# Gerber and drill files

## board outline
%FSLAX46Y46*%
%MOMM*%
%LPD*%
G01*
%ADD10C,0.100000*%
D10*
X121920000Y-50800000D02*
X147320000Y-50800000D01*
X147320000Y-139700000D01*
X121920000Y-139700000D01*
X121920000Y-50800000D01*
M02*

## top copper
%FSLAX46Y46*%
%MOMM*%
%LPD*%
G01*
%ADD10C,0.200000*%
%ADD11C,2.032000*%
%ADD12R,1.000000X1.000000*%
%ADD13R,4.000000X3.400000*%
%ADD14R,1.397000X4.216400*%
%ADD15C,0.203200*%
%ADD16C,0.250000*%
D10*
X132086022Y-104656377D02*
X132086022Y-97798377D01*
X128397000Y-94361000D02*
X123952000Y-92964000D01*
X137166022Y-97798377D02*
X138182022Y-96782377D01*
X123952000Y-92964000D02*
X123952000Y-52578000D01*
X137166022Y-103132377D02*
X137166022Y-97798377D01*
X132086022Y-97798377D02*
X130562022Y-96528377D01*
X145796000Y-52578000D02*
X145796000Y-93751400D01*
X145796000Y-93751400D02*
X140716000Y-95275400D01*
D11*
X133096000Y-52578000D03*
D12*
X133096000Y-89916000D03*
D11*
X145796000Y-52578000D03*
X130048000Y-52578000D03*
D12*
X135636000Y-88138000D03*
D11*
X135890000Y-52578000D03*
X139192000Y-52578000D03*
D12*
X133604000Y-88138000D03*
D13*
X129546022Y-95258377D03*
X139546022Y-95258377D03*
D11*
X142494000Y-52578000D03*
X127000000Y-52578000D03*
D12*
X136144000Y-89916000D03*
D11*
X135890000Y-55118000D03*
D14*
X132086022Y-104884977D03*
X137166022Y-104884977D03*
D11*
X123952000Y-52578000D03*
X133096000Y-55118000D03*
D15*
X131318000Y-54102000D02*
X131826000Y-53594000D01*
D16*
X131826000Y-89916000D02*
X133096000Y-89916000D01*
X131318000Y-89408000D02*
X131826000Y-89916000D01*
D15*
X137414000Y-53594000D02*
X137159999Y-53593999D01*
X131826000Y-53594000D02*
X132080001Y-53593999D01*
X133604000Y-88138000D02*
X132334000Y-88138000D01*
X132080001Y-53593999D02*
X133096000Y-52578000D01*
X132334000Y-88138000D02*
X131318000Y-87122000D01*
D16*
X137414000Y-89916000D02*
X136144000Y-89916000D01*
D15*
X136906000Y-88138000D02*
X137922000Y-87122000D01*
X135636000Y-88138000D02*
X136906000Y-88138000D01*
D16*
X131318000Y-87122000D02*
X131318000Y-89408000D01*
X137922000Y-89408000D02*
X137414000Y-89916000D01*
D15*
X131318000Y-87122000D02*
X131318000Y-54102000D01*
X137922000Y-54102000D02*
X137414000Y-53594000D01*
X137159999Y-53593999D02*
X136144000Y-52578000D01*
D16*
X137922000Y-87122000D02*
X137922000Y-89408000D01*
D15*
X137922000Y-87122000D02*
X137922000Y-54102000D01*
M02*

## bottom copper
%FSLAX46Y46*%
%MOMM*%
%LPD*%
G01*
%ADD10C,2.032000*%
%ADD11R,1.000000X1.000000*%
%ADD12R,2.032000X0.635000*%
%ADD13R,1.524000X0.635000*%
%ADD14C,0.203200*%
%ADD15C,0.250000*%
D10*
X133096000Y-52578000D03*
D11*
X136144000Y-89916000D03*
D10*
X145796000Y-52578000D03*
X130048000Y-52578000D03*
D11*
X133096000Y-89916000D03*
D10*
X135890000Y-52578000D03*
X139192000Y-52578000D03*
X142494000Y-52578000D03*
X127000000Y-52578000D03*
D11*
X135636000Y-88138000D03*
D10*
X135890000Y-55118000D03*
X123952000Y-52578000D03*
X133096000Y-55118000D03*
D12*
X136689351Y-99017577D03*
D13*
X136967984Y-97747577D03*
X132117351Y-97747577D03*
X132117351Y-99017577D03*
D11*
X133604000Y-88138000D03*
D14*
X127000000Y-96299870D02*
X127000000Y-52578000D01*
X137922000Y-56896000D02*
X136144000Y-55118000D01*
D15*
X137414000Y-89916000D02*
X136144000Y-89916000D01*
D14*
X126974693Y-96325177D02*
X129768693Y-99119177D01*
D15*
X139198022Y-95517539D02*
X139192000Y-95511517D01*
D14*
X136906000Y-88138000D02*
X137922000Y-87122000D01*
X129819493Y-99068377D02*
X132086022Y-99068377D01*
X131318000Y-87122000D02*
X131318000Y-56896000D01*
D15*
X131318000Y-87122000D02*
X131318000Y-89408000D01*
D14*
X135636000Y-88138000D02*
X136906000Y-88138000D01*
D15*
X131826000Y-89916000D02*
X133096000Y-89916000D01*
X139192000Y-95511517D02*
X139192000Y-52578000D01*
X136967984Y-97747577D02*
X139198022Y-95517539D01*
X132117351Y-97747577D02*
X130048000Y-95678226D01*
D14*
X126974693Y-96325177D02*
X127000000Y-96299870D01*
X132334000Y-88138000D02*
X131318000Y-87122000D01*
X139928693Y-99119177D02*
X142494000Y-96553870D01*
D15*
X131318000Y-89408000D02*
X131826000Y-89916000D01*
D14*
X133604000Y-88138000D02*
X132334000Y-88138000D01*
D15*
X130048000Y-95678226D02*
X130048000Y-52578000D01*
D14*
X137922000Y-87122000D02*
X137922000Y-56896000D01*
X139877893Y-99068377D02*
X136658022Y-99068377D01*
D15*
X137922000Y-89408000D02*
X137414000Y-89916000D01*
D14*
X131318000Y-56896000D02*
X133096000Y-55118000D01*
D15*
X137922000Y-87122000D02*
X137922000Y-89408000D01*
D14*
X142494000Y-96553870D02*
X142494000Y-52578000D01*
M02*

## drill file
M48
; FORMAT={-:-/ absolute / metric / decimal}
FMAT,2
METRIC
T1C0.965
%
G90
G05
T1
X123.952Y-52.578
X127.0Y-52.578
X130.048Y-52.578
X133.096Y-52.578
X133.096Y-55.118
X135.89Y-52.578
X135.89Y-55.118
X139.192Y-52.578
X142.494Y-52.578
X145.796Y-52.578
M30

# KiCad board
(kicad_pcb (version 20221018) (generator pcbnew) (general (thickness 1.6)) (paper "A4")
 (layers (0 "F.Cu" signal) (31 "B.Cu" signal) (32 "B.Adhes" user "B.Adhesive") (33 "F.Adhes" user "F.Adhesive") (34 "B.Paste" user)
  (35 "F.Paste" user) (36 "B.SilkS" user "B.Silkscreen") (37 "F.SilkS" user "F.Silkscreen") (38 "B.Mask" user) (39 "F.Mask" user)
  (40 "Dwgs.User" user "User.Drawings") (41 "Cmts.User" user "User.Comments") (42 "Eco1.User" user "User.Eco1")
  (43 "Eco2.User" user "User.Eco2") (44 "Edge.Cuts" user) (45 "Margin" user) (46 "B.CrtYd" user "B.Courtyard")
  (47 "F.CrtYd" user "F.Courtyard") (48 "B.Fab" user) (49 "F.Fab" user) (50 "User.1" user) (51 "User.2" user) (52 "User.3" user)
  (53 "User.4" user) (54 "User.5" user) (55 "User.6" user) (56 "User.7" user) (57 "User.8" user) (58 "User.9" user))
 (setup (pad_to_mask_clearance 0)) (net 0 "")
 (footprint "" (layer "F.Cu") (at 133.096 52.578)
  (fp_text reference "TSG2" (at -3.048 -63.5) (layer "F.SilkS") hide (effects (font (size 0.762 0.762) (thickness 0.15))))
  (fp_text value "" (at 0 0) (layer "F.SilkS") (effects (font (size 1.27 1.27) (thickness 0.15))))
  (pad "1" thru_hole circle (at 0 0) (size 2.032 2.032) (drill 0.9652) (layers "*.Cu" "*.Mask")))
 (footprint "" (layer "F.Cu") (at 133.096 89.916)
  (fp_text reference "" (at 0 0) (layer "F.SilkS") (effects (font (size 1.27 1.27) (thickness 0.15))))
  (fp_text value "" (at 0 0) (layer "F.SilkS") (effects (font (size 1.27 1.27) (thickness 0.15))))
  (pad "1" smd rect (at 0 0) (size 1 1) (layers "F.Cu" "F.Mask")))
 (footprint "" (layer "F.Cu") (at 136.144 89.916)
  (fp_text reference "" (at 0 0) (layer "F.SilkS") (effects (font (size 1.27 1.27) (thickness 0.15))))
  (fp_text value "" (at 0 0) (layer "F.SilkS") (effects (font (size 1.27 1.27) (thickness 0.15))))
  (pad "1" smd rect (at 0 0 180) (size 1 1) (layers "B.Cu" "B.Mask")))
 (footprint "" (layer "F.Cu") (at 145.796 66.04)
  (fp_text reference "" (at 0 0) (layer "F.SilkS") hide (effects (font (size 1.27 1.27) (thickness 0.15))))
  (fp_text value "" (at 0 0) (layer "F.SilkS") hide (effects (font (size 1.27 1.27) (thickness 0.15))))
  (pad "1" thru_hole circle (at 0 -13.462) (size 2.032 2.032) (drill 0.9652) (layers "*.Cu" "*.Mask")))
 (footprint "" (layer "F.Cu") (at 130.048 66.04)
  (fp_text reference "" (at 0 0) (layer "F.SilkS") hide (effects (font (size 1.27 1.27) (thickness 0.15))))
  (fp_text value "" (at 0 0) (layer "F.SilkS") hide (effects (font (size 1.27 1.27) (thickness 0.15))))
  (pad "1" thru_hole circle (at 0 -13.462) (size 2.032 2.032) (drill 0.9652) (layers "*.Cu" "*.Mask")))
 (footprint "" (layer "F.Cu") (at 133.096 89.916)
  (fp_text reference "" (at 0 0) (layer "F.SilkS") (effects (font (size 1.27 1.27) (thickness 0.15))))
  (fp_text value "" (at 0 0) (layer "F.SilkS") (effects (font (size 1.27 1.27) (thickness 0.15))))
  (pad "1" smd rect (at 0 0 180) (size 1 1) (layers "B.Cu" "B.Mask")))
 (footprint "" (layer "F.Cu") (at 135.636 88.138)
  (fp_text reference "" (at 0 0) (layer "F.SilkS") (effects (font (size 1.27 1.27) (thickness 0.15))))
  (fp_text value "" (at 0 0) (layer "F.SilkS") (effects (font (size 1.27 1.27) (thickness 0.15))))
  (pad "1" smd rect (at 0 0) (size 1 1) (layers "F.Cu" "F.Mask")))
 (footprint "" (layer "F.Cu") (at 135.89 52.578)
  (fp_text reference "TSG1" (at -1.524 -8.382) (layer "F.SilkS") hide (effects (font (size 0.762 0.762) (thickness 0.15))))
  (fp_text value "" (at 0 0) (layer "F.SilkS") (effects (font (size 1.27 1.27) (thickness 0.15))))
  (pad "1" thru_hole circle (at 0 0) (size 2.032 2.032) (drill 0.9652) (layers "*.Cu" "*.Mask")))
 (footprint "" (layer "F.Cu") (at 139.192 66.04)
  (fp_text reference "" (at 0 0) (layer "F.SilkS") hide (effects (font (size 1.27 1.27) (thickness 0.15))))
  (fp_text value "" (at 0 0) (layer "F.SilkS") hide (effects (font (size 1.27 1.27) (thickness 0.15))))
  (pad "1" thru_hole circle (at 0 -13.462) (size 2.032 2.032) (drill 0.9652) (layers "*.Cu" "*.Mask")))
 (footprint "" (layer "F.Cu") (at 133.604 75.438)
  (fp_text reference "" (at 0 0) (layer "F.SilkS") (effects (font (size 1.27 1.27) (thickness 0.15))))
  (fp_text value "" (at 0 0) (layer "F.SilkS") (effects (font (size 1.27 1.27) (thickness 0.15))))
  (pad "1" smd rect (at 0 12.7) (size 1 1) (layers "F.Cu" "F.Mask")))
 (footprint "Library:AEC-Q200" (layer "F.Cu") (at 134.626022 101.608377)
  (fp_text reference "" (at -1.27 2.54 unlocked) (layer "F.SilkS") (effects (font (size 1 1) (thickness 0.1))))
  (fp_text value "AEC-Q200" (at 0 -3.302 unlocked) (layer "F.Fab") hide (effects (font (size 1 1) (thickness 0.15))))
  (pad "1" smd rect (at -5.08 -6.35 180) (size 4 3.4) (layers "F.Cu" "F.Mask"))
  (pad "2" smd rect (at 4.92 -6.35 180) (size 4 3.4) (layers "F.Cu" "F.Mask")))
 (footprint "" (layer "F.Cu") (at 142.494 66.04)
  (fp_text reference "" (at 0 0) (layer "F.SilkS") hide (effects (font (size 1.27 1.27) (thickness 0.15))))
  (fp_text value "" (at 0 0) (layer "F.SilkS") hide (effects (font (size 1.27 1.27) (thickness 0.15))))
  (pad "1" thru_hole circle (at 0 -13.462) (size 2.032 2.032) (drill 0.9652) (layers "*.Cu" "*.Mask")))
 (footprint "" (layer "F.Cu") (at 127 66.04)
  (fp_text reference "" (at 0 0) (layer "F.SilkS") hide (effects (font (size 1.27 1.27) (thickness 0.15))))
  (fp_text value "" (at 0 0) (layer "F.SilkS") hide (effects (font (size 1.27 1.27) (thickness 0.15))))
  (pad "1" thru_hole circle (at 0 -13.462) (size 2.032 2.032) (drill 0.9652) (layers "*.Cu" "*.Mask")))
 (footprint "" (layer "F.Cu") (at 135.636 88.138)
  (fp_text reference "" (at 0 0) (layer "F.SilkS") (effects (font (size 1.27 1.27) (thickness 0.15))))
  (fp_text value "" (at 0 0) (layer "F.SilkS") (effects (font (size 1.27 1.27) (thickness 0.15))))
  (pad "1" smd rect (at 0 0 180) (size 1 1) (layers "B.Cu" "B.Mask")))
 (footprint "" (layer "F.Cu") (at 136.144 89.916)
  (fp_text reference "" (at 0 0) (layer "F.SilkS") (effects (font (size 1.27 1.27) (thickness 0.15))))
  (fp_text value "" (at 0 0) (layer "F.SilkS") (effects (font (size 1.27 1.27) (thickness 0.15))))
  (pad "1" smd rect (at 0 0) (size 1 1) (layers "F.Cu" "F.Mask")))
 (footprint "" (layer "F.Cu") (at 135.89 55.118)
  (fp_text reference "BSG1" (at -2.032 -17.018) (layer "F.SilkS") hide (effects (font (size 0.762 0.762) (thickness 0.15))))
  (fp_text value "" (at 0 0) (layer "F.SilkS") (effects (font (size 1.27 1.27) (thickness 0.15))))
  (pad "1" thru_hole circle (at 0 0) (size 2.032 2.032) (drill 0.9652) (layers "*.Cu" "*.Mask")))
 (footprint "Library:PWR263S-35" (layer "F.Cu") (at 135.896022 105.926377)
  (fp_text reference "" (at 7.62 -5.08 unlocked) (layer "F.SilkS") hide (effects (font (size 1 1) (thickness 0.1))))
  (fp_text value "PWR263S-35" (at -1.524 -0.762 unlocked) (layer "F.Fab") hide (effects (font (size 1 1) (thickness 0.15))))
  (pad "1" smd rect (at -3.81 -1.0414) (size 1.397 4.2164) (layers "F.Cu" "F.Mask"))
  (pad "2" smd rect (at 1.27 -1.0414) (size 1.397 4.2164) (layers "F.Cu" "F.Mask")))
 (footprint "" (layer "F.Cu") (at 123.952 66.04)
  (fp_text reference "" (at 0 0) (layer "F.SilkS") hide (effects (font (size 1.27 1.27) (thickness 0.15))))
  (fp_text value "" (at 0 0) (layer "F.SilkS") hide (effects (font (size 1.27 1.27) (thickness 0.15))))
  (pad "1" thru_hole circle (at 0 -13.462) (size 2.032 2.032) (drill 0.9652) (layers "*.Cu" "*.Mask")))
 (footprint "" (layer "F.Cu") (at 133.096 55.118)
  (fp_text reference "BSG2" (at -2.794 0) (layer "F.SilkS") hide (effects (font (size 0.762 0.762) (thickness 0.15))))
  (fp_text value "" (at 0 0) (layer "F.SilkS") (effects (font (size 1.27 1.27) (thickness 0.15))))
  (pad "1" thru_hole circle (at 0 0) (size 2.032 2.032) (drill 0.9652) (layers "*.Cu" "*.Mask")))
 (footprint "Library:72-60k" (layer "B.Cu") (at 132.879351 102.827577 180)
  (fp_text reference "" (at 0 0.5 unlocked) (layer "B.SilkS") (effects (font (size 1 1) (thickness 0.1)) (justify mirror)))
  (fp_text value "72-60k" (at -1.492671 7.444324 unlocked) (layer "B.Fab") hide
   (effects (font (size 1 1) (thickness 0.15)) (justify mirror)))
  (pad "1" smd rect (at -3.81 3.81) (size 2.032 0.635) (layers "B.Cu" "B.Mask"))
  (pad "2" smd rect (at -4.088633 5.08) (size 1.524 0.635) (layers "B.Cu" "B.Mask"))
  (pad "3" smd rect (at 0.762 5.08) (size 1.524 0.635) (layers "B.Cu" "B.Mask"))
  (pad "4" smd rect (at 0.762 3.81) (size 1.524 0.635) (layers "B.Cu" "B.Mask")))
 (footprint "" (layer "B.Cu") (at 133.604 75.438 180)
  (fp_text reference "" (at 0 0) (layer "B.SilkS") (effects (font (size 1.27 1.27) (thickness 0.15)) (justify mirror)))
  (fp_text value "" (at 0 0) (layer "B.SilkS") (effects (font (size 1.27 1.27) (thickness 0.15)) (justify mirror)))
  (pad "1" smd rect (at 0 -12.7 180) (size 1 1) (layers "B.Cu" "B.Mask")))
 (gr_line (start 132.086022 104.656377) (end 132.086022 97.798377) (stroke (width 0.2) (type default)) (layer "F.Cu"))
 (gr_line (start 128.397 94.361) (end 123.952 92.964) (stroke (width 0.2) (type default)) (layer "F.Cu"))
 (gr_line (start 137.166022 97.798377) (end 138.182022 96.782377) (stroke (width 0.2) (type default)) (layer "F.Cu"))
 (gr_line (start 123.952 92.964) (end 123.952 52.578) (stroke (width 0.2) (type default)) (layer "F.Cu"))
 (gr_line (start 137.166022 103.132377) (end 137.166022 97.798377) (stroke (width 0.2) (type default)) (layer "F.Cu"))
 (gr_line (start 132.086022 97.798377) (end 130.562022 96.528377) (stroke (width 0.2) (type default)) (layer "F.Cu"))
 (gr_line (start 145.796 52.578) (end 145.796 93.7514) (stroke (width 0.2) (type default)) (layer "F.Cu"))
 (gr_line (start 145.796 93.7514) (end 140.716 95.2754) (stroke (width 0.2) (type default)) (layer "F.Cu"))
 (gr_rect (start 121.92 50.8) (end 147.32 139.7) (stroke (width 0.1) (type default)) (fill none) (layer "Edge.Cuts"))
 (segment (start 131.318 54.102) (end 131.826 53.594) (width 0.2032) (layer "F.Cu") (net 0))
 (segment (start 131.826 89.916) (end 133.096 89.916) (width 0.25) (layer "F.Cu") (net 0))
 (segment (start 131.318 89.408) (end 131.826 89.916) (width 0.25) (layer "F.Cu") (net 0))
 (segment (start 137.414 53.594) (end 137.159999 53.593999) (width 0.2032) (layer "F.Cu") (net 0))
 (segment (start 131.826 53.594) (end 132.080001 53.593999) (width 0.2032) (layer "F.Cu") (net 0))
 (segment (start 133.604 88.138) (end 132.334 88.138) (width 0.2032) (layer "F.Cu") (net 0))
 (segment (start 132.080001 53.593999) (end 133.096 52.578) (width 0.2032) (layer "F.Cu") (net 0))
 (segment (start 132.334 88.138) (end 131.318 87.122) (width 0.2032) (layer "F.Cu") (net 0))
 (segment (start 137.414 89.916) (end 136.144 89.916) (width 0.25) (layer "F.Cu") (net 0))
 (segment (start 136.906 88.138) (end 137.922 87.122) (width 0.2032) (layer "F.Cu") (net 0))
 (segment (start 135.636 88.138) (end 136.906 88.138) (width 0.2032) (layer "F.Cu") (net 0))
 (segment (start 131.318 87.122) (end 131.318 89.408) (width 0.25) (layer "F.Cu") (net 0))
 (segment (start 137.922 89.408) (end 137.414 89.916) (width 0.25) (layer "F.Cu") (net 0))
 (segment (start 131.318 87.122) (end 131.318 54.102) (width 0.2032) (layer "F.Cu") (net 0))
 (segment (start 137.922 54.102) (end 137.414 53.594) (width 0.2032) (layer "F.Cu") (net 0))
 (segment (start 137.159999 53.593999) (end 136.144 52.578) (width 0.2032) (layer "F.Cu") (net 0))
 (segment (start 137.922 87.122) (end 137.922 89.408) (width 0.25) (layer "F.Cu") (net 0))
 (segment (start 137.922 87.122) (end 137.922 54.102) (width 0.2032) (layer "F.Cu") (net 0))
 (segment (start 127 96.29987) (end 127 52.578) (width 0.2032) (layer "B.Cu") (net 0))
 (segment (start 137.922 56.896) (end 136.144 55.118) (width 0.2032) (layer "B.Cu") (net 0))
 (segment (start 137.414 89.916) (end 136.144 89.916) (width 0.25) (layer "B.Cu") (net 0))
 (segment (start 126.974693 96.325177) (end 129.768693 99.119177) (width 0.2032) (layer "B.Cu") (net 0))
 (segment (start 139.198022 95.517539) (end 139.192 95.511517) (width 0.25) (layer "B.Cu") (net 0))
 (segment (start 136.906 88.138) (end 137.922 87.122) (width 0.2032) (layer "B.Cu") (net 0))
 (segment (start 129.819493 99.068377) (end 132.086022 99.068377) (width 0.2032) (layer "B.Cu") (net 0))
 (segment (start 131.318 87.122) (end 131.318 56.896) (width 0.2032) (layer "B.Cu") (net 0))
 (segment (start 131.318 87.122) (end 131.318 89.408) (width 0.25) (layer "B.Cu") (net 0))
 (segment (start 135.636 88.138) (end 136.906 88.138) (width 0.2032) (layer "B.Cu") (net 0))
 (segment (start 131.826 89.916) (end 133.096 89.916) (width 0.25) (layer "B.Cu") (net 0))
 (segment (start 139.192 95.511517) (end 139.192 52.578) (width 0.25) (layer "B.Cu") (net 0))
 (segment (start 136.967984 97.747577) (end 139.198022 95.517539) (width 0.25) (layer "B.Cu") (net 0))
 (segment (start 132.117351 97.747577) (end 130.048 95.678226) (width 0.25) (layer "B.Cu") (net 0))
 (segment (start 126.974693 96.325177) (end 127 96.29987) (width 0.2032) (layer "B.Cu") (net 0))
 (segment (start 132.334 88.138) (end 131.318 87.122) (width 0.2032) (layer "B.Cu") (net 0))
 (segment (start 139.928693 99.119177) (end 142.494 96.55387) (width 0.2032) (layer "B.Cu") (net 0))
 (segment (start 131.318 89.408) (end 131.826 89.916) (width 0.25) (layer "B.Cu") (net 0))
 (segment (start 133.604 88.138) (end 132.334 88.138) (width 0.2032) (layer "B.Cu") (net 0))
 (segment (start 130.048 95.678226) (end 130.048 52.578) (width 0.25) (layer "B.Cu") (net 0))
 (segment (start 137.922 87.122) (end 137.922 56.896) (width 0.2032) (layer "B.Cu") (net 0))
 (segment (start 139.877893 99.068377) (end 136.658022 99.068377) (width 0.2032) (layer "B.Cu") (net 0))
 (segment (start 137.922 89.408) (end 137.414 89.916) (width 0.25) (layer "B.Cu") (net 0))
 (segment (start 131.318 56.896) (end 133.096 55.118) (width 0.2032) (layer "B.Cu") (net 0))
 (segment (start 137.922 87.122) (end 137.922 89.408) (width 0.25) (layer "B.Cu") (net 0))
 (segment (start 142.494 96.55387) (end 142.494 52.578) (width 0.2032) (layer "B.Cu") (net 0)))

